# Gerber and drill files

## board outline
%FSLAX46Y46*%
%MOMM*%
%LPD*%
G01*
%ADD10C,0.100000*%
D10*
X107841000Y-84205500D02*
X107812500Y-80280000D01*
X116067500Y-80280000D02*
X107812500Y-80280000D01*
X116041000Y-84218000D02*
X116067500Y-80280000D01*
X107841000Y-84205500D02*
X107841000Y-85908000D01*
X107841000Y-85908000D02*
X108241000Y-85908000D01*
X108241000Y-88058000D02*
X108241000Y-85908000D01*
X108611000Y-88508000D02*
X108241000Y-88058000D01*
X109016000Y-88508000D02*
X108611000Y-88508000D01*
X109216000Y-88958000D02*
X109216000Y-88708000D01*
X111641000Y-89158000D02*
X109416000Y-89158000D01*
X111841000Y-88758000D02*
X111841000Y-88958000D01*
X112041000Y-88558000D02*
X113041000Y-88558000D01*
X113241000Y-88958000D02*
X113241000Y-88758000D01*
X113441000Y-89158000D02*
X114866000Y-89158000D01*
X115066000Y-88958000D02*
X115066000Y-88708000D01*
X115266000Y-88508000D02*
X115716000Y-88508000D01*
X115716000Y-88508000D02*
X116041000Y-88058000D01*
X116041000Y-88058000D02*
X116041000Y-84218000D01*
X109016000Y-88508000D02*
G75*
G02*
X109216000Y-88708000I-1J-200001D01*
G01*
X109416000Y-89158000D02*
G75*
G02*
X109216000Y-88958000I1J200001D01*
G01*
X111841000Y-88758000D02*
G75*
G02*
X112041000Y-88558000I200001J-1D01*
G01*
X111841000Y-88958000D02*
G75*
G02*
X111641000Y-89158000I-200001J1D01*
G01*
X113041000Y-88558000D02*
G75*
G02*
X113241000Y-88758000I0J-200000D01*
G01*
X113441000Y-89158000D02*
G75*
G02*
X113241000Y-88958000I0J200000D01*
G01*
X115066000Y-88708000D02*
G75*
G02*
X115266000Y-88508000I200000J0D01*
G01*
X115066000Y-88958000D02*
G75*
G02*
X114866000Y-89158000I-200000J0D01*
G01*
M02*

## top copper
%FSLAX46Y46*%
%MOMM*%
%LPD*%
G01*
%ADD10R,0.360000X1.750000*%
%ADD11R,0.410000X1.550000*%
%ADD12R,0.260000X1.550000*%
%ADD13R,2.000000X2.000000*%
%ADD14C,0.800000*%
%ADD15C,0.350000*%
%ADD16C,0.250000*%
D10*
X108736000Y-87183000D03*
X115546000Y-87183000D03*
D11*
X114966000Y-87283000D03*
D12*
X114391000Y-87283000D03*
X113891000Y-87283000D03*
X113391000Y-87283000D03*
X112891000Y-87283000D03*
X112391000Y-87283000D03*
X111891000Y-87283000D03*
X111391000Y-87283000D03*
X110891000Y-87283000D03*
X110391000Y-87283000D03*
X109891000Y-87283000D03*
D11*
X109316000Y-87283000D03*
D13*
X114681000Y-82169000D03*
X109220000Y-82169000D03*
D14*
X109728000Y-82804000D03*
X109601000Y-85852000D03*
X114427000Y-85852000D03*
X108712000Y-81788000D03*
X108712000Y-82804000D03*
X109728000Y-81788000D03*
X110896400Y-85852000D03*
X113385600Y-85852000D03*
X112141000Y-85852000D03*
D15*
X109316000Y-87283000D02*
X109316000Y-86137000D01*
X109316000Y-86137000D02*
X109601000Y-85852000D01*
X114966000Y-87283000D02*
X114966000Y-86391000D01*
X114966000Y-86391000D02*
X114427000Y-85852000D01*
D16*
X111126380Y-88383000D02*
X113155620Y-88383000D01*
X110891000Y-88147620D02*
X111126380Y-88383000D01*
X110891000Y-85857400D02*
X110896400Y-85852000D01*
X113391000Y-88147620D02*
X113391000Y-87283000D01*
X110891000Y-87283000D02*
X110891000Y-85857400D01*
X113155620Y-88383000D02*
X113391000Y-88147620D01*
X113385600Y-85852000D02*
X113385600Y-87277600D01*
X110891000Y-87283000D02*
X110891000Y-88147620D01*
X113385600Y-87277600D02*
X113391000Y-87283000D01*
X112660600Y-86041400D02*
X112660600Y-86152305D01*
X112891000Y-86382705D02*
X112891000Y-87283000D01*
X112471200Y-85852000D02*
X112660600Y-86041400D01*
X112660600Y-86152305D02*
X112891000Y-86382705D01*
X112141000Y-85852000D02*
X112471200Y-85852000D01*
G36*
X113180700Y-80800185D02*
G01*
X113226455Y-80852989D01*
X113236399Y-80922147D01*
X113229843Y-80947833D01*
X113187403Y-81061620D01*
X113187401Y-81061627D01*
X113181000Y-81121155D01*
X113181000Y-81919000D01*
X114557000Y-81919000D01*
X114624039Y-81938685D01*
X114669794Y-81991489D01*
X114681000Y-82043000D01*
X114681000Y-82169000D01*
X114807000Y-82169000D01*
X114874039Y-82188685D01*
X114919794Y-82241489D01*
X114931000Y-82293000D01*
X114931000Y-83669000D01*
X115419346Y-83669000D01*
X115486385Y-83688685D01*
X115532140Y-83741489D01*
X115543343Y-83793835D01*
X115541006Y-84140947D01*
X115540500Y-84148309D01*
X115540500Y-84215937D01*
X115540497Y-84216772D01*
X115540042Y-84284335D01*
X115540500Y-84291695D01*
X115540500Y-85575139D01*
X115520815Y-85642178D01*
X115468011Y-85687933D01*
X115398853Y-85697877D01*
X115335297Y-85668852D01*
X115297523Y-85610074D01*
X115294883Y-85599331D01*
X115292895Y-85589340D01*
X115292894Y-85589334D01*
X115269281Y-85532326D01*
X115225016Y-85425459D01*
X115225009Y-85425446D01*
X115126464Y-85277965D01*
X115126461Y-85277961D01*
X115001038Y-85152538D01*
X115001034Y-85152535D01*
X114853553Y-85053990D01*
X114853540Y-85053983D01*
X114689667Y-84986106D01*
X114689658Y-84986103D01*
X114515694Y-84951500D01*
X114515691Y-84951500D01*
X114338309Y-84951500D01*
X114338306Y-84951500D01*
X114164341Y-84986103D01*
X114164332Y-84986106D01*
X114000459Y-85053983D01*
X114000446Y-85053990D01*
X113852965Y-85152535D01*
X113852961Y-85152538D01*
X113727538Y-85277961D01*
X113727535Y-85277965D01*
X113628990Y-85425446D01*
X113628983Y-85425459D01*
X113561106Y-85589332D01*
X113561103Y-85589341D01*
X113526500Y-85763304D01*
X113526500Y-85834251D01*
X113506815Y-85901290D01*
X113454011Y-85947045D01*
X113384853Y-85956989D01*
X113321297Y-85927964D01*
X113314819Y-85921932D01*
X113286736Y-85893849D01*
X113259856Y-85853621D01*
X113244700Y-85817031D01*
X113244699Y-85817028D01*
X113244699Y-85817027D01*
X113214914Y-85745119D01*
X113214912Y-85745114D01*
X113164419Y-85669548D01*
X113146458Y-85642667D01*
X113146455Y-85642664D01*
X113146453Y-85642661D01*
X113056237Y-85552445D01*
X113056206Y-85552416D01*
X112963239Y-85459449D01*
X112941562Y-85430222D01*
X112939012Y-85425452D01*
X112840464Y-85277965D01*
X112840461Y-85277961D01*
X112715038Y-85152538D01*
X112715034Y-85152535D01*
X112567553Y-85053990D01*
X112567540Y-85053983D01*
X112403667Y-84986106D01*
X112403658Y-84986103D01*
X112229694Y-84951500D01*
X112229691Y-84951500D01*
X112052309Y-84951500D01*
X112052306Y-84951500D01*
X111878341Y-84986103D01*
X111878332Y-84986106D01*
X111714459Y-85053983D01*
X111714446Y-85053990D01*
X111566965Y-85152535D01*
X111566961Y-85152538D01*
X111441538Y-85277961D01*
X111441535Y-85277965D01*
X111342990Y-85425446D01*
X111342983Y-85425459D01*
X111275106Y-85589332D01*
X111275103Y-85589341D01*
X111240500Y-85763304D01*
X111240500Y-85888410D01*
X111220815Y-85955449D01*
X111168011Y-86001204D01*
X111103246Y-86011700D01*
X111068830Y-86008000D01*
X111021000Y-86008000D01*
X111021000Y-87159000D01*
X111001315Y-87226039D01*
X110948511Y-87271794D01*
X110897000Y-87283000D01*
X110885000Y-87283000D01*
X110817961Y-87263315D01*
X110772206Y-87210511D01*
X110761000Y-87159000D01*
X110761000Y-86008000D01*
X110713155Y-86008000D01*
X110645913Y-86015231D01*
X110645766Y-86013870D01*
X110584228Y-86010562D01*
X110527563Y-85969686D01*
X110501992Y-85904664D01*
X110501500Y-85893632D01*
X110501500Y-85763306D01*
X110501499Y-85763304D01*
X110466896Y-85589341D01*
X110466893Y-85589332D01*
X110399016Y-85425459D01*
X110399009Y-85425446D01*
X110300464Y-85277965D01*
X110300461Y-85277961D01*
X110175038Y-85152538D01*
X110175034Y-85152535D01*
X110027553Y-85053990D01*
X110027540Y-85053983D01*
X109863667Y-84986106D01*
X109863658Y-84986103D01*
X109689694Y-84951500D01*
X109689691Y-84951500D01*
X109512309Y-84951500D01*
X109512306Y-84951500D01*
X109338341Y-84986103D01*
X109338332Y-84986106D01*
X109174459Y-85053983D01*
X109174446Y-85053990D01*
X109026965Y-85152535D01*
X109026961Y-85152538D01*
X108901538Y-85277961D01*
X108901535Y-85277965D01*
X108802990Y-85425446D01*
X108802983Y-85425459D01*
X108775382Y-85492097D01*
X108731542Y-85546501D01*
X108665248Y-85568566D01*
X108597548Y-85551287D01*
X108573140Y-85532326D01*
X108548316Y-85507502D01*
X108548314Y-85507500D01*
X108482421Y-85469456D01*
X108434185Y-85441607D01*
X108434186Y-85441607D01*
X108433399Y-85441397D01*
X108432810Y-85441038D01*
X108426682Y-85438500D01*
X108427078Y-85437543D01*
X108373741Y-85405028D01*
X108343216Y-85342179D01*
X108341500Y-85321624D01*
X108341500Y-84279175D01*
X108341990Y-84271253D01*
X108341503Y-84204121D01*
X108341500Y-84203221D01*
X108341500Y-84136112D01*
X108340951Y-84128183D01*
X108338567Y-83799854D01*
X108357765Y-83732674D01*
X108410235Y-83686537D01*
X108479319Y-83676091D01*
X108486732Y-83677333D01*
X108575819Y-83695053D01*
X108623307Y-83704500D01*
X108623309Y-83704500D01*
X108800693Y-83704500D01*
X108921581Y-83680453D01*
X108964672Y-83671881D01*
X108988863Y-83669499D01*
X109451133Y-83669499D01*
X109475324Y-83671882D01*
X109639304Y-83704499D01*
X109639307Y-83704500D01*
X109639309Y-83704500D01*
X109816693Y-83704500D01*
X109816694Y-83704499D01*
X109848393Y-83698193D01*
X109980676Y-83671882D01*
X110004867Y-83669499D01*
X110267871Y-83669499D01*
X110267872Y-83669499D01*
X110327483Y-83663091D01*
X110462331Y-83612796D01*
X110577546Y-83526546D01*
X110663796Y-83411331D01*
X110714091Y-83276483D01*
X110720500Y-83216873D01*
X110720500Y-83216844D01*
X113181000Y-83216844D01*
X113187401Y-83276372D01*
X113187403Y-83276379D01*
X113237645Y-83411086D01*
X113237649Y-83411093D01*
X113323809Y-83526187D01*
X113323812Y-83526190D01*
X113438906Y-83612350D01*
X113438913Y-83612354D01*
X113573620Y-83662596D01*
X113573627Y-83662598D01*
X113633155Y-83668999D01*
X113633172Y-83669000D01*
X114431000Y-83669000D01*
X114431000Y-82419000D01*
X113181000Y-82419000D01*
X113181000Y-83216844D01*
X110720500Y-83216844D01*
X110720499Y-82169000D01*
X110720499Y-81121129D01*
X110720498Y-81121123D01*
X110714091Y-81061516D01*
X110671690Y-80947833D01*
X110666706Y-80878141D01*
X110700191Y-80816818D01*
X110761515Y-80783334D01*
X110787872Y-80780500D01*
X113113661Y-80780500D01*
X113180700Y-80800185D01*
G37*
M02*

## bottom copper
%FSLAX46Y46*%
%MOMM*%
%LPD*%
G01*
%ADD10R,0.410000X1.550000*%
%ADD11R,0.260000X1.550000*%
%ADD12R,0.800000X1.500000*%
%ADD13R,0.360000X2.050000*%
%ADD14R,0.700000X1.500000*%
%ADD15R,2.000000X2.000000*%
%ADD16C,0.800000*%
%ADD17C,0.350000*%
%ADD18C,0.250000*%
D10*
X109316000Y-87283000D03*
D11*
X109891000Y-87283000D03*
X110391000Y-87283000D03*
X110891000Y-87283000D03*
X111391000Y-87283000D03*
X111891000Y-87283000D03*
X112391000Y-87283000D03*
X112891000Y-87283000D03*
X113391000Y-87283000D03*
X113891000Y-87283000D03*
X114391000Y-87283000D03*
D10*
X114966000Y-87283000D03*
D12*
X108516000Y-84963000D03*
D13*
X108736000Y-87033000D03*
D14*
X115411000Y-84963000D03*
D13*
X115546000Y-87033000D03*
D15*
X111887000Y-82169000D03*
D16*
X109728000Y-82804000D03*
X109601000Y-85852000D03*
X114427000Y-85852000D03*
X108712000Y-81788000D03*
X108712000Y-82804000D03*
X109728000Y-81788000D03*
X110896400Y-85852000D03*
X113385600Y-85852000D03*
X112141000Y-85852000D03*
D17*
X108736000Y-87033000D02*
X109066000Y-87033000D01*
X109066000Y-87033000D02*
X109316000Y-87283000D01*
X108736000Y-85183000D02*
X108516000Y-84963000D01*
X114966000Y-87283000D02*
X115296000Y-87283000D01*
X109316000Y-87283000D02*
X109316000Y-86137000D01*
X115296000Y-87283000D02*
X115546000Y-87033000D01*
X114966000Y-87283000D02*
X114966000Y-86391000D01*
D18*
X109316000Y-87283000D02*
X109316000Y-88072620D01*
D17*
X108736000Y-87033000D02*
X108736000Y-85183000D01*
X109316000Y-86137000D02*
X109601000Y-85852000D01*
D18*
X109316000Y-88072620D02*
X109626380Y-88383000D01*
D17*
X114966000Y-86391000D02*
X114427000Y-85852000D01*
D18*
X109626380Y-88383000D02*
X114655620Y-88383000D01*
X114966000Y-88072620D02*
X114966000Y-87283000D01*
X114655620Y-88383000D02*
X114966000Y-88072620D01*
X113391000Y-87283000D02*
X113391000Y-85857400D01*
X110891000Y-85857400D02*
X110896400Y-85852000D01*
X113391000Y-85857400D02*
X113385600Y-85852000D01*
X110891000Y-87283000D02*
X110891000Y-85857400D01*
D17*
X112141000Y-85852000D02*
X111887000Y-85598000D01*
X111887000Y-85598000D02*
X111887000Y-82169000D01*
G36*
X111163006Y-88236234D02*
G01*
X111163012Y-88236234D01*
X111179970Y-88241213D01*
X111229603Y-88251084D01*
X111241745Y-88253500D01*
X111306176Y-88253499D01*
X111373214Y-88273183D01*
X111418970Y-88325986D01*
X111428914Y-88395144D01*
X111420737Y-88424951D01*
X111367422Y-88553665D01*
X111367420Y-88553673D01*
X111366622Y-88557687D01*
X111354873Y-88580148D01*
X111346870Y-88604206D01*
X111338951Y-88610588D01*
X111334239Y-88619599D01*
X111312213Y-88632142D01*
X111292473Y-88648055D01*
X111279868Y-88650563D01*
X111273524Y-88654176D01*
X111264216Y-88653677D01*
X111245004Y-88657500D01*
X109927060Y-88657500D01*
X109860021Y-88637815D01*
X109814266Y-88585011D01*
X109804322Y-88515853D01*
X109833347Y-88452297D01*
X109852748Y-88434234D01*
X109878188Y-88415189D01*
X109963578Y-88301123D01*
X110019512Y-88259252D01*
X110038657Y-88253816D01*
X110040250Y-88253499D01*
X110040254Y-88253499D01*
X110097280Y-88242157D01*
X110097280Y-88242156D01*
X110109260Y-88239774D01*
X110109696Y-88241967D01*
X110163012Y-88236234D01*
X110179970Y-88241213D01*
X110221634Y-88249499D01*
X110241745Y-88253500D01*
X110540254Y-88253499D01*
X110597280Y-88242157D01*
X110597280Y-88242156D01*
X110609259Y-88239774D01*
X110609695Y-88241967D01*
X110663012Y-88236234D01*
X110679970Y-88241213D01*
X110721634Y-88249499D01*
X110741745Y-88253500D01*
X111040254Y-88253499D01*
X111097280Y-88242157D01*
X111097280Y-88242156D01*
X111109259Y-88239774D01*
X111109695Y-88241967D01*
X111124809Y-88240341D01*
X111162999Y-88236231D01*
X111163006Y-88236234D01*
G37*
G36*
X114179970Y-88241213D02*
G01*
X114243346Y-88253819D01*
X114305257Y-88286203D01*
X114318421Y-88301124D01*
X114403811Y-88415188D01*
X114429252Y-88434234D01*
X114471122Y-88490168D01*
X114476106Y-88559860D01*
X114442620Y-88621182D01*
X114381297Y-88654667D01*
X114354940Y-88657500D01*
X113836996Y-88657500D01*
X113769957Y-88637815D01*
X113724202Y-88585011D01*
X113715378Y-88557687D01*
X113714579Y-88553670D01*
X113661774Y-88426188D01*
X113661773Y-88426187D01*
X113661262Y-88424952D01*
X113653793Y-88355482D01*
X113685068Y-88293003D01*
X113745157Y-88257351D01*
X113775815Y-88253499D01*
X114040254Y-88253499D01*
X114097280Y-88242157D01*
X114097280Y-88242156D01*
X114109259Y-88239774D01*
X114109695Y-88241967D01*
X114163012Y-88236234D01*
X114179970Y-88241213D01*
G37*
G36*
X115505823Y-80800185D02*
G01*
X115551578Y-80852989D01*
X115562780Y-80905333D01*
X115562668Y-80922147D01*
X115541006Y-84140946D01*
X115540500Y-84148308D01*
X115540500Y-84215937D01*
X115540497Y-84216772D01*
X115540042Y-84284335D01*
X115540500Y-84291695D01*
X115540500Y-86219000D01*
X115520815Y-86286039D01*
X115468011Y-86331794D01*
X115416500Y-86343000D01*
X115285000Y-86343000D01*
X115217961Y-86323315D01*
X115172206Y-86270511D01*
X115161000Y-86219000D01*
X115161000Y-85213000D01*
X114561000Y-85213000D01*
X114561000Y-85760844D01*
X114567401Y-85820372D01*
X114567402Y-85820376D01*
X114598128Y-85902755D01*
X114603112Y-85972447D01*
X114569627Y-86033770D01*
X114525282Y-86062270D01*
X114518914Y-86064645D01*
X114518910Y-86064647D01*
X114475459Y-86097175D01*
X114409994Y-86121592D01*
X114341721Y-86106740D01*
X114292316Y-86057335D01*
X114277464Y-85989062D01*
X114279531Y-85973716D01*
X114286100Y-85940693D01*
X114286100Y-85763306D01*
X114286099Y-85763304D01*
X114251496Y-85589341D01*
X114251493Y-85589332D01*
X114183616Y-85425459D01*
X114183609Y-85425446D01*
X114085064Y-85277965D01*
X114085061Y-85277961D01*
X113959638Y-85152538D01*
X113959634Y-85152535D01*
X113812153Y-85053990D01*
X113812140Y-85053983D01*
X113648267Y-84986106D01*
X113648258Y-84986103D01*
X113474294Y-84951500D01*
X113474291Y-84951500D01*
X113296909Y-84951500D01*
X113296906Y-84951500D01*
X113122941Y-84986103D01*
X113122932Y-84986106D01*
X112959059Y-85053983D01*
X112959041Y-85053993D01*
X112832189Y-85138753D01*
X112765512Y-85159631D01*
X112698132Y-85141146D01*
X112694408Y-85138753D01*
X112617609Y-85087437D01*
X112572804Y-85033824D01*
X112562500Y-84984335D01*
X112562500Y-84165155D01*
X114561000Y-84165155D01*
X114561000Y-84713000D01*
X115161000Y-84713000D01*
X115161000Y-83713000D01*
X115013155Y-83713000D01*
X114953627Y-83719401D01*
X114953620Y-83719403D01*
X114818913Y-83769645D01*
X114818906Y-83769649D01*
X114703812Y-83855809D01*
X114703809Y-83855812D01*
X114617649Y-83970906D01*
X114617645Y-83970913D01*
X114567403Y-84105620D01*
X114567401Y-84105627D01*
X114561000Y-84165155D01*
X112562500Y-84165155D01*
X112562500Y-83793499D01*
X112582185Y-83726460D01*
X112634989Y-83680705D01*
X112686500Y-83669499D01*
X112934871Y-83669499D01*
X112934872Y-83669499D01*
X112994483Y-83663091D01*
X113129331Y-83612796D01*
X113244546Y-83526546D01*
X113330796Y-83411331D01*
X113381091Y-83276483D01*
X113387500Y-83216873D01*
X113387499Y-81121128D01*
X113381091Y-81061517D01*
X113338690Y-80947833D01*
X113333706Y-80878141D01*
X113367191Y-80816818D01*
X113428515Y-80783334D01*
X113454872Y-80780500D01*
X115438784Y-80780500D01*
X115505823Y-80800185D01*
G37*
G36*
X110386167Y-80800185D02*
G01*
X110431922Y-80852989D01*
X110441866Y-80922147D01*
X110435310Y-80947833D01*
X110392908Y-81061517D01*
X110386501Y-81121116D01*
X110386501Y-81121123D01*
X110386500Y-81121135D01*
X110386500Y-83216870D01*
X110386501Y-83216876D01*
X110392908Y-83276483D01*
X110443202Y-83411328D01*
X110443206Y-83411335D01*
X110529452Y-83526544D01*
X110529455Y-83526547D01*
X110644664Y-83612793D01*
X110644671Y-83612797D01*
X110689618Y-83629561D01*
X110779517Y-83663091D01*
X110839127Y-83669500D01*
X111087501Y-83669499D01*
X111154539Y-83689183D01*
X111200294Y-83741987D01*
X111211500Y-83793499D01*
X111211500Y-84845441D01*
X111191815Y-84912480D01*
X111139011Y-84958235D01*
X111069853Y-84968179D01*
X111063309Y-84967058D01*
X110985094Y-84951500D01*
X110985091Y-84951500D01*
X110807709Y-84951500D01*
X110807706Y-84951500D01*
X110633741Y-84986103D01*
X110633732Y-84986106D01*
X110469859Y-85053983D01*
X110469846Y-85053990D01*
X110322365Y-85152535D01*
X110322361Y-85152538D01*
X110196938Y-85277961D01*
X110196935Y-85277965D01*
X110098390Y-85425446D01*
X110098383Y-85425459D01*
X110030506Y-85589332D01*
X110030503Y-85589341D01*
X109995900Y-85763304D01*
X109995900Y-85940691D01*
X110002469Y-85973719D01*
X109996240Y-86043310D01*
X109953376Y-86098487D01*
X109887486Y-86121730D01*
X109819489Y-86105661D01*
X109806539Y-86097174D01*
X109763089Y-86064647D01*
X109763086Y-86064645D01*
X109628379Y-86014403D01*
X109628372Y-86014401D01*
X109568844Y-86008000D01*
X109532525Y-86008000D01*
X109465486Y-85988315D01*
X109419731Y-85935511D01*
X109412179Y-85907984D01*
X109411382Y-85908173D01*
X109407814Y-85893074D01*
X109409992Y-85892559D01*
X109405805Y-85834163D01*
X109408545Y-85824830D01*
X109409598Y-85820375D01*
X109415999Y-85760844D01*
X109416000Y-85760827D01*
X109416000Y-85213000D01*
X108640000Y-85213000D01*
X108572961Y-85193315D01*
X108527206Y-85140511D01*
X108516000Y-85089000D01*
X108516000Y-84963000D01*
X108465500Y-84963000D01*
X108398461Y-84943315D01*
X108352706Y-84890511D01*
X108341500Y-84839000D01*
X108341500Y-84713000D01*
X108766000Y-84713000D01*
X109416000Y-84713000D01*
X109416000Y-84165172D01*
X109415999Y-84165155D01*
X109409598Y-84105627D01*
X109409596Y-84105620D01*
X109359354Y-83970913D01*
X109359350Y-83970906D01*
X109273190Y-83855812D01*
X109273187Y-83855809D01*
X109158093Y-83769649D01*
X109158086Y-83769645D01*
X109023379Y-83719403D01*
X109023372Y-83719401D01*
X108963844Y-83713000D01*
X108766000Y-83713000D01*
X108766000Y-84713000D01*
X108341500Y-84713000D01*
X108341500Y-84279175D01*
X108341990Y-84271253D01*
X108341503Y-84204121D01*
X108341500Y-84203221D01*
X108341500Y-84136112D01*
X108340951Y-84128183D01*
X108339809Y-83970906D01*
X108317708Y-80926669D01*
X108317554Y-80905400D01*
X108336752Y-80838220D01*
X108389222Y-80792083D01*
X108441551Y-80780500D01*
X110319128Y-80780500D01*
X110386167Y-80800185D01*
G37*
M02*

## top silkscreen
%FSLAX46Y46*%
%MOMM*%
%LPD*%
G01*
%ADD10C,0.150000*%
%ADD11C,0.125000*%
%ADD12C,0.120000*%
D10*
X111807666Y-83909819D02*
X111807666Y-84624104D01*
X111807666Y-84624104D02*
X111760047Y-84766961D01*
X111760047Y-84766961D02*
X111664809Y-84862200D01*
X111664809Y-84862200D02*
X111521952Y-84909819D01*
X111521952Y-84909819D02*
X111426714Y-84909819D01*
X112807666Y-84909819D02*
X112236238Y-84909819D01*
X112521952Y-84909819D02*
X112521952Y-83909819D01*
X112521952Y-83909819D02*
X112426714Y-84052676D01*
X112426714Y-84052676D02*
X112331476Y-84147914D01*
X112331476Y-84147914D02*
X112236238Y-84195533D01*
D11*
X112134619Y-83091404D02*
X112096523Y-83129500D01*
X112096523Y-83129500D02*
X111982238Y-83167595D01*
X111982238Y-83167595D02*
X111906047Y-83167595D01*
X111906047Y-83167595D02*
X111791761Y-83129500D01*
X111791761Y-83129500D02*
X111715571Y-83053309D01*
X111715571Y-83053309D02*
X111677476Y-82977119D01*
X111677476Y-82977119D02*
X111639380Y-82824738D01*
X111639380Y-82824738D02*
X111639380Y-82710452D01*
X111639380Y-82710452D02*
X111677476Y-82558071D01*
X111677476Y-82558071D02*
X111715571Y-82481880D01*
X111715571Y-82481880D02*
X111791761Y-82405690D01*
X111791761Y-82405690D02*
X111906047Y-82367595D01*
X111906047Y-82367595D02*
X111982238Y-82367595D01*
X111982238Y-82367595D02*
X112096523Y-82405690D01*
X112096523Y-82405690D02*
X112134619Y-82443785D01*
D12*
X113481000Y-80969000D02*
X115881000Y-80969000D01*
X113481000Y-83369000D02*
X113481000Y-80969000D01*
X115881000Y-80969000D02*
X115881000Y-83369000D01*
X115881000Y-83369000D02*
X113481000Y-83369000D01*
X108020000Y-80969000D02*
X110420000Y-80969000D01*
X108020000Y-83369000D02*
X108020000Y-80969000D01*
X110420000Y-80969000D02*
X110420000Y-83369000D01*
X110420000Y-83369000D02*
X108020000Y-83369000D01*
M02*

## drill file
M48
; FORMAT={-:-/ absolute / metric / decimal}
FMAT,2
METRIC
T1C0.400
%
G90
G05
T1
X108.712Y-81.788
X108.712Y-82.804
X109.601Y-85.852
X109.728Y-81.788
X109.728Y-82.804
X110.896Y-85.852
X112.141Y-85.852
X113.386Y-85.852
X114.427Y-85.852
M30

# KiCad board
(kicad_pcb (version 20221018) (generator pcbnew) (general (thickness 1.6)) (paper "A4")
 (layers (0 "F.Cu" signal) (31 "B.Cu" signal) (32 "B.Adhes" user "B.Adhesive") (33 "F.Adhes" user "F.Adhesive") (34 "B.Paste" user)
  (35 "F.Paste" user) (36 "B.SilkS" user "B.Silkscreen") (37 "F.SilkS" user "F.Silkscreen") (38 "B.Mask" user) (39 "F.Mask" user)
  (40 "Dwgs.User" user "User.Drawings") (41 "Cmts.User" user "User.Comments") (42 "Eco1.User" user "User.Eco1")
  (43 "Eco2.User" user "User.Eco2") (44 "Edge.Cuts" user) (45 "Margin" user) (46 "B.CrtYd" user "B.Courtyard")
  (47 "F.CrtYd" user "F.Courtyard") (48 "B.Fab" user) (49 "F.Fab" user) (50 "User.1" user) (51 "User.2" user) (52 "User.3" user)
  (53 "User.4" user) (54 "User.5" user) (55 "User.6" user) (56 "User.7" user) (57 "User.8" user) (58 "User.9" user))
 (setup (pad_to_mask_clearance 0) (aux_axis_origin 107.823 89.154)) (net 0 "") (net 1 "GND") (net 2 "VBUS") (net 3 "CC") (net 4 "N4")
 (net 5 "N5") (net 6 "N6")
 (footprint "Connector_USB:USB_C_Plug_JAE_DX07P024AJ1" (layer "F.Cu") (at 112.141 86.1355) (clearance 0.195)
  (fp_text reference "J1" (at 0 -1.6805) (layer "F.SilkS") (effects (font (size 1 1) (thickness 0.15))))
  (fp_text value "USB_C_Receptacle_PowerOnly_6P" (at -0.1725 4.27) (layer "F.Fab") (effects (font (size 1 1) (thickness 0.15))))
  (fp_line (start -4.3 -1.93) (end -4.3 -0.2275) (stroke (width 0.1) (type solid)) (layer "Edge.Cuts"))
  (fp_line (start -4.3 -0.2275) (end -3.9 -0.2275) (stroke (width 0.1) (type solid)) (layer "Edge.Cuts"))
  (fp_line (start -3.9 1.9225) (end -3.9 -0.2275) (stroke (width 0.1) (type solid)) (layer "Edge.Cuts"))
  (fp_line (start -3.53 2.3725) (end -3.9 1.9225) (stroke (width 0.1) (type solid)) (layer "Edge.Cuts"))
  (fp_line (start -3.125 2.3725) (end -3.53 2.3725) (stroke (width 0.1) (type solid)) (layer "Edge.Cuts"))
  (fp_line (start -2.925 2.8225) (end -2.925 2.5725) (stroke (width 0.1) (type solid)) (layer "Edge.Cuts"))
  (fp_line (start -0.5 3.0225) (end -2.725 3.0225) (stroke (width 0.1) (type solid)) (layer "Edge.Cuts"))
  (fp_line (start -0.3 2.6225) (end -0.3 2.8225) (stroke (width 0.1) (type solid)) (layer "Edge.Cuts"))
  (fp_line (start -0.1 2.4225) (end 0.9 2.4225) (stroke (width 0.1) (type solid)) (layer "Edge.Cuts"))
  (fp_line (start 1.1 2.8225) (end 1.1 2.6225) (stroke (width 0.1) (type solid)) (layer "Edge.Cuts"))
  (fp_line (start 1.3 3.0225) (end 2.725 3.0225) (stroke (width 0.1) (type solid)) (layer "Edge.Cuts"))
  (fp_line (start 2.925 2.8225) (end 2.925 2.5725) (stroke (width 0.1) (type solid)) (layer "Edge.Cuts"))
  (fp_line (start 3.125 2.3725) (end 3.575 2.3725) (stroke (width 0.1) (type solid)) (layer "Edge.Cuts"))
  (fp_line (start 3.575 2.3725) (end 3.9 1.9225) (stroke (width 0.1) (type solid)) (layer "Edge.Cuts"))
  (fp_line (start 3.9 1.9225) (end 3.9 -1.9175) (stroke (width 0.1) (type solid)) (layer "Edge.Cuts"))
  (fp_arc (start -3.125 2.3725) (mid -2.983579 2.431079) (end -2.925 2.5725) (stroke (width 0.1) (type solid)) (layer "Edge.Cuts"))
  (fp_arc (start -2.725 3.0225) (mid -2.866421 2.963921) (end -2.925 2.8225) (stroke (width 0.1) (type solid)) (layer "Edge.Cuts"))
  (fp_arc (start -0.3 2.6225) (mid -0.241421 2.481079) (end -0.1 2.4225) (stroke (width 0.1) (type solid)) (layer "Edge.Cuts"))
  (fp_arc (start -0.3 2.8225) (mid -0.358579 2.963921) (end -0.5 3.0225) (stroke (width 0.1) (type solid)) (layer "Edge.Cuts"))
  (fp_arc (start 0.9 2.4225) (mid 1.041421 2.481079) (end 1.1 2.6225) (stroke (width 0.1) (type solid)) (layer "Edge.Cuts"))
  (fp_arc (start 1.3 3.0225) (mid 1.158579 2.963921) (end 1.1 2.8225) (stroke (width 0.1) (type solid)) (layer "Edge.Cuts"))
  (fp_arc (start 2.925 2.5725) (mid 2.983579 2.431079) (end 3.125 2.3725) (stroke (width 0.1) (type solid)) (layer "Edge.Cuts"))
  (fp_arc (start 2.925 2.8225) (mid 2.866421 2.963921) (end 2.725 3.0225) (stroke (width 0.1) (type solid)) (layer "Edge.Cuts"))
  (pad "" smd rect (at -3.405 1.0475) (size 0.36 1.75) (layers "F.Cu" "F.Mask"))
  (pad "" smd rect (at 3.405 1.0475) (size 0.36 1.75) (layers "F.Cu" "F.Mask"))
  (pad "A1" smd rect (at 2.825 1.1475) (size 0.41 1.55) (layers "F.Cu" "F.Paste" "F.Mask") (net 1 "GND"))
  (pad "A2" smd rect (at 2.25 1.1475) (size 0.26 1.55) (layers "F.Cu" "F.Paste" "F.Mask"))
  (pad "A3" smd rect (at 1.75 1.1475) (size 0.26 1.55) (layers "F.Cu" "F.Paste" "F.Mask"))
  (pad "A4" smd rect (at 1.25 1.1475) (size 0.26 1.55) (layers "F.Cu" "F.Paste" "F.Mask") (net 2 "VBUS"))
  (pad "A5" smd rect (at 0.75 1.1475) (size 0.26 1.55) (layers "F.Cu" "F.Paste" "F.Mask") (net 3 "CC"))
  (pad "A6" smd rect (at 0.25 1.1475 180) (size 0.26 1.55) (layers "F.Cu" "F.Paste" "F.Mask") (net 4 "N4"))
  (pad "A7" smd rect (at -0.25 1.1475 180) (size 0.26 1.55) (layers "F.Cu" "F.Paste" "F.Mask") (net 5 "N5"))
  (pad "A8" smd rect (at -0.75 1.1475) (size 0.26 1.55) (layers "F.Cu" "F.Paste" "F.Mask"))
  (pad "A9" smd rect (at -1.25 1.1475) (size 0.26 1.55) (layers "F.Cu" "F.Paste" "F.Mask") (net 2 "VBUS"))
  (pad "A10" smd rect (at -1.75 1.1475) (size 0.26 1.55) (layers "F.Cu" "F.Paste" "F.Mask"))
  (pad "A11" smd rect (at -2.25 1.1475) (size 0.26 1.55) (layers "F.Cu" "F.Paste" "F.Mask"))
  (pad "A12" smd rect (at -2.825 1.1475) (size 0.41 1.55) (layers "F.Cu" "F.Paste" "F.Mask") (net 1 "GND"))
  (pad "B1" smd rect (at -2.825 1.1475) (size 0.41 1.55) (layers "B.Cu" "B.Paste" "B.Mask") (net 1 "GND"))
  (pad "B2" smd rect (at -2.25 1.1475) (size 0.26 1.55) (layers "B.Cu" "B.Paste" "B.Mask"))
  (pad "B3" smd rect (at -1.75 1.1475) (size 0.26 1.55) (layers "B.Cu" "B.Paste" "B.Mask"))
  (pad "B4" smd rect (at -1.25 1.1475) (size 0.26 1.55) (layers "B.Cu" "B.Paste" "B.Mask") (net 2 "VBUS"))
  (pad "B5" smd rect (at -0.75 1.1475) (size 0.26 1.55) (layers "B.Cu" "B.Paste" "B.Mask") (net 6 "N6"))
  (pad "B6" smd rect (at -0.25 1.1475 180) (size 0.26 1.55) (layers "B.Cu" "B.Paste" "B.Mask"))
  (pad "B7" smd rect (at 0.25 1.1475) (size 0.26 1.55) (layers "B.Cu" "B.Paste" "B.Mask"))
  (pad "B8" smd rect (at 0.75 1.1475) (size 0.26 1.55) (layers "B.Cu" "B.Paste" "B.Mask"))
  (pad "B9" smd rect (at 1.25 1.1475) (size 0.26 1.55) (layers "B.Cu" "B.Paste" "B.Mask") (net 2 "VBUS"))
  (pad "B10" smd rect (at 1.75 1.1475) (size 0.26 1.55) (layers "B.Cu" "B.Paste" "B.Mask"))
  (pad "B11" smd rect (at 2.25 1.1475) (size 0.26 1.55) (layers "B.Cu" "B.Paste" "B.Mask"))
  (pad "B12" smd rect (at 2.825 1.1475) (size 0.41 1.55) (layers "B.Cu" "B.Paste" "B.Mask") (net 1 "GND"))
  (pad "S1" smd rect (at -3.625 -1.1725) (size 0.8 1.5) (layers "B.Cu" "B.Paste" "B.Mask") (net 1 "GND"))
  (pad "S1" smd rect (at -3.405 0.8975) (size 0.36 2.05) (layers "B.Cu" "B.Paste" "B.Mask") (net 1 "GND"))
  (pad "S1" smd rect (at 3.27 -1.1725 180) (size 0.7 1.5) (layers "B.Cu" "B.Paste" "B.Mask") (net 1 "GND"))
  (pad "S1" smd rect (at 3.405 0.8975) (size 0.36 2.05) (layers "B.Cu" "B.Paste" "B.Mask") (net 1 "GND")))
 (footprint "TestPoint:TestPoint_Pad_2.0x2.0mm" (layer "F.Cu") (at 114.681 82.169)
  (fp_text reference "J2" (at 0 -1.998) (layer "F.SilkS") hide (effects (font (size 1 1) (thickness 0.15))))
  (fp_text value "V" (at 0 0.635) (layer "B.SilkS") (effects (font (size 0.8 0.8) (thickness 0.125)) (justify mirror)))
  (fp_line (start -1.2 -1.2) (end 1.2 -1.2) (stroke (width 0.12) (type solid)) (layer "F.SilkS"))
  (fp_line (start -1.2 1.2) (end -1.2 -1.2) (stroke (width 0.12) (type solid)) (layer "F.SilkS"))
  (fp_line (start 1.2 -1.2) (end 1.2 1.2) (stroke (width 0.12) (type solid)) (layer "F.SilkS"))
  (fp_line (start 1.2 1.2) (end -1.2 1.2) (stroke (width 0.12) (type solid)) (layer "F.SilkS"))
  (pad "1" smd rect (at 0 0) (size 2 2) (layers "F.Cu" "F.Mask") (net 2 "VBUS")))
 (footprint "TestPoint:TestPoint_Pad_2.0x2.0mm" (layer "F.Cu") (at 109.22 82.169)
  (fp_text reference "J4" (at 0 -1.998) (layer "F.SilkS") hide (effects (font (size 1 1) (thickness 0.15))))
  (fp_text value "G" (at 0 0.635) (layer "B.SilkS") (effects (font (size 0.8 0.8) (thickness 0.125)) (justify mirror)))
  (fp_line (start -1.2 -1.2) (end 1.2 -1.2) (stroke (width 0.12) (type solid)) (layer "F.SilkS"))
  (fp_line (start -1.2 1.2) (end -1.2 -1.2) (stroke (width 0.12) (type solid)) (layer "F.SilkS"))
  (fp_line (start 1.2 -1.2) (end 1.2 1.2) (stroke (width 0.12) (type solid)) (layer "F.SilkS"))
  (fp_line (start 1.2 1.2) (end -1.2 1.2) (stroke (width 0.12) (type solid)) (layer "F.SilkS"))
  (pad "1" smd rect (at 0 0) (size 2 2) (layers "F.Cu" "F.Mask") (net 1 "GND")))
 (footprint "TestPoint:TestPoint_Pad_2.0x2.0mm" (layer "B.Cu") (at 111.887 82.169 180)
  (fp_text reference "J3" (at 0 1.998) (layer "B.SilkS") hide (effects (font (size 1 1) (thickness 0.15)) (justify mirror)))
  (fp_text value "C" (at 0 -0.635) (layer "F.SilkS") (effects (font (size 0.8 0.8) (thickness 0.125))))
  (pad "1" smd rect (at 0 0 180) (size 2 2) (layers "B.Cu" "B.Mask") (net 3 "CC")))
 (gr_line (start 107.841 84.2055) (end 107.8125 80.28) (stroke (width 0.1) (type default)) (layer "Edge.Cuts"))
 (gr_line (start 116.0675 80.28) (end 107.8125 80.28) (stroke (width 0.1) (type default)) (layer "Edge.Cuts"))
 (gr_line (start 116.041 84.218) (end 116.0675 80.28) (stroke (width 0.1) (type default)) (layer "Edge.Cuts"))
 (segment (start 109.316 87.283) (end 109.316 86.137) (width 0.35) (layer "F.Cu") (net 1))
 (segment (start 109.316 86.137) (end 109.601 85.852) (width 0.35) (layer "F.Cu") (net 1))
 (segment (start 114.966 87.283) (end 114.966 86.391) (width 0.35) (layer "F.Cu") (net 1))
 (segment (start 114.966 86.391) (end 114.427 85.852) (width 0.35) (layer "F.Cu") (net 1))
 (via (at 109.728 82.804) (size 0.8) (drill 0.4) (layers "F.Cu" "B.Cu") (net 1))
 (via (at 109.601 85.852) (size 0.8) (drill 0.4) (layers "F.Cu" "B.Cu") (free) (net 1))
 (via (at 114.427 85.852) (size 0.8) (drill 0.4) (layers "F.Cu" "B.Cu") (free) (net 1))
 (via (at 108.712 81.788) (size 0.8) (drill 0.4) (layers "F.Cu" "B.Cu") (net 1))
 (via (at 108.712 82.804) (size 0.8) (drill 0.4) (layers "F.Cu" "B.Cu") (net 1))
 (via (at 109.728 81.788) (size 0.8) (drill 0.4) (layers "F.Cu" "B.Cu") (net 1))
 (segment (start 108.736 87.033) (end 109.066 87.033) (width 0.35) (layer "B.Cu") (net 1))
 (segment (start 109.066 87.033) (end 109.316 87.283) (width 0.35) (layer "B.Cu") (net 1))
 (segment (start 108.736 85.183) (end 108.516 84.963) (width 0.35) (layer "B.Cu") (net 1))
 (segment (start 114.966 87.283) (end 115.296 87.283) (width 0.35) (layer "B.Cu") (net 1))
 (segment (start 109.316 87.283) (end 109.316 86.137) (width 0.35) (layer "B.Cu") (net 1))
 (segment (start 115.296 87.283) (end 115.546 87.033) (width 0.35) (layer "B.Cu") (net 1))
 (segment (start 114.966 87.283) (end 114.966 86.391) (width 0.35) (layer "B.Cu") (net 1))
 (segment (start 109.316 87.283) (end 109.316 88.07262) (width 0.25) (layer "B.Cu") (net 1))
 (segment (start 108.736 87.033) (end 108.736 85.183) (width 0.35) (layer "B.Cu") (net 1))
 (segment (start 109.316 86.137) (end 109.601 85.852) (width 0.35) (layer "B.Cu") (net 1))
 (segment (start 109.316 88.07262) (end 109.62638 88.383) (width 0.25) (layer "B.Cu") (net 1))
 (segment (start 114.966 86.391) (end 114.427 85.852) (width 0.35) (layer "B.Cu") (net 1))
 (segment (start 109.62638 88.383) (end 114.65562 88.383) (width 0.25) (layer "B.Cu") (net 1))
 (segment (start 114.966 88.07262) (end 114.966 87.283) (width 0.25) (layer "B.Cu") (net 1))
 (segment (start 114.65562 88.383) (end 114.966 88.07262) (width 0.25) (layer "B.Cu") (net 1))
 (segment (start 111.12638 88.383) (end 113.15562 88.383) (width 0.25) (layer "F.Cu") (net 2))
 (segment (start 110.891 88.14762) (end 111.12638 88.383) (width 0.25) (layer "F.Cu") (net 2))
 (segment (start 110.891 85.8574) (end 110.8964 85.852) (width 0.25) (layer "F.Cu") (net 2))
 (segment (start 113.391 88.14762) (end 113.391 87.283) (width 0.25) (layer "F.Cu") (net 2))
 (segment (start 110.891 87.283) (end 110.891 85.8574) (width 0.25) (layer "F.Cu") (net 2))
 (segment (start 113.15562 88.383) (end 113.391 88.14762) (width 0.25) (layer "F.Cu") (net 2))
 (segment (start 113.3856 85.852) (end 113.3856 87.2776) (width 0.25) (layer "F.Cu") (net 2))
 (segment (start 110.891 87.283) (end 110.891 88.14762) (width 0.25) (layer "F.Cu") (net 2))
 (segment (start 113.3856 87.2776) (end 113.391 87.283) (width 0.25) (layer "F.Cu") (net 2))
 (via (at 110.8964 85.852) (size 0.8) (drill 0.4) (layers "F.Cu" "B.Cu") (free) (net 2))
 (via (at 113.3856 85.852) (size 0.8) (drill 0.4) (layers "F.Cu" "B.Cu") (free) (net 2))
 (segment (start 113.391 87.283) (end 113.391 85.8574) (width 0.25) (layer "B.Cu") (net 2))
 (segment (start 110.891 85.8574) (end 110.8964 85.852) (width 0.25) (layer "B.Cu") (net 2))
 (segment (start 113.391 85.8574) (end 113.3856 85.852) (width 0.25) (layer "B.Cu") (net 2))
 (segment (start 110.891 87.283) (end 110.891 85.8574) (width 0.25) (layer "B.Cu") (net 2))
 (segment (start 112.6606 86.0414) (end 112.6606 86.152305) (width 0.25) (layer "F.Cu") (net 3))
 (segment (start 112.891 86.382705) (end 112.891 87.283) (width 0.25) (layer "F.Cu") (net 3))
 (segment (start 112.4712 85.852) (end 112.6606 86.0414) (width 0.25) (layer "F.Cu") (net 3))
 (segment (start 112.6606 86.152305) (end 112.891 86.382705) (width 0.25) (layer "F.Cu") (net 3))
 (segment (start 112.141 85.852) (end 112.4712 85.852) (width 0.25) (layer "F.Cu") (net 3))
 (via (at 112.141 85.852) (size 0.8) (drill 0.4) (layers "F.Cu" "B.Cu") (free) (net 3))
 (segment (start 112.141 85.852) (end 111.887 85.598) (width 0.35) (layer "B.Cu") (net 3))
 (segment (start 111.887 85.598) (end 111.887 82.169) (width 0.35) (layer "B.Cu") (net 3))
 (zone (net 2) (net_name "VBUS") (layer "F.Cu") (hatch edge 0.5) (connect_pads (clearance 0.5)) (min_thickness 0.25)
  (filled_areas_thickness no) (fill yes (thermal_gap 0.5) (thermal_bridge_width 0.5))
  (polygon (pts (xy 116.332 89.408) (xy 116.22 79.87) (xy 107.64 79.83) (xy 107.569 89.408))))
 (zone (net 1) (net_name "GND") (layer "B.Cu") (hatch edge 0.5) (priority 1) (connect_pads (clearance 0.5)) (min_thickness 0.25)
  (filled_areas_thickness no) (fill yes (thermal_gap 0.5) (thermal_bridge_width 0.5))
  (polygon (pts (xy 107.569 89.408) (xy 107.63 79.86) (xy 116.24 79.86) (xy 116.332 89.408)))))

